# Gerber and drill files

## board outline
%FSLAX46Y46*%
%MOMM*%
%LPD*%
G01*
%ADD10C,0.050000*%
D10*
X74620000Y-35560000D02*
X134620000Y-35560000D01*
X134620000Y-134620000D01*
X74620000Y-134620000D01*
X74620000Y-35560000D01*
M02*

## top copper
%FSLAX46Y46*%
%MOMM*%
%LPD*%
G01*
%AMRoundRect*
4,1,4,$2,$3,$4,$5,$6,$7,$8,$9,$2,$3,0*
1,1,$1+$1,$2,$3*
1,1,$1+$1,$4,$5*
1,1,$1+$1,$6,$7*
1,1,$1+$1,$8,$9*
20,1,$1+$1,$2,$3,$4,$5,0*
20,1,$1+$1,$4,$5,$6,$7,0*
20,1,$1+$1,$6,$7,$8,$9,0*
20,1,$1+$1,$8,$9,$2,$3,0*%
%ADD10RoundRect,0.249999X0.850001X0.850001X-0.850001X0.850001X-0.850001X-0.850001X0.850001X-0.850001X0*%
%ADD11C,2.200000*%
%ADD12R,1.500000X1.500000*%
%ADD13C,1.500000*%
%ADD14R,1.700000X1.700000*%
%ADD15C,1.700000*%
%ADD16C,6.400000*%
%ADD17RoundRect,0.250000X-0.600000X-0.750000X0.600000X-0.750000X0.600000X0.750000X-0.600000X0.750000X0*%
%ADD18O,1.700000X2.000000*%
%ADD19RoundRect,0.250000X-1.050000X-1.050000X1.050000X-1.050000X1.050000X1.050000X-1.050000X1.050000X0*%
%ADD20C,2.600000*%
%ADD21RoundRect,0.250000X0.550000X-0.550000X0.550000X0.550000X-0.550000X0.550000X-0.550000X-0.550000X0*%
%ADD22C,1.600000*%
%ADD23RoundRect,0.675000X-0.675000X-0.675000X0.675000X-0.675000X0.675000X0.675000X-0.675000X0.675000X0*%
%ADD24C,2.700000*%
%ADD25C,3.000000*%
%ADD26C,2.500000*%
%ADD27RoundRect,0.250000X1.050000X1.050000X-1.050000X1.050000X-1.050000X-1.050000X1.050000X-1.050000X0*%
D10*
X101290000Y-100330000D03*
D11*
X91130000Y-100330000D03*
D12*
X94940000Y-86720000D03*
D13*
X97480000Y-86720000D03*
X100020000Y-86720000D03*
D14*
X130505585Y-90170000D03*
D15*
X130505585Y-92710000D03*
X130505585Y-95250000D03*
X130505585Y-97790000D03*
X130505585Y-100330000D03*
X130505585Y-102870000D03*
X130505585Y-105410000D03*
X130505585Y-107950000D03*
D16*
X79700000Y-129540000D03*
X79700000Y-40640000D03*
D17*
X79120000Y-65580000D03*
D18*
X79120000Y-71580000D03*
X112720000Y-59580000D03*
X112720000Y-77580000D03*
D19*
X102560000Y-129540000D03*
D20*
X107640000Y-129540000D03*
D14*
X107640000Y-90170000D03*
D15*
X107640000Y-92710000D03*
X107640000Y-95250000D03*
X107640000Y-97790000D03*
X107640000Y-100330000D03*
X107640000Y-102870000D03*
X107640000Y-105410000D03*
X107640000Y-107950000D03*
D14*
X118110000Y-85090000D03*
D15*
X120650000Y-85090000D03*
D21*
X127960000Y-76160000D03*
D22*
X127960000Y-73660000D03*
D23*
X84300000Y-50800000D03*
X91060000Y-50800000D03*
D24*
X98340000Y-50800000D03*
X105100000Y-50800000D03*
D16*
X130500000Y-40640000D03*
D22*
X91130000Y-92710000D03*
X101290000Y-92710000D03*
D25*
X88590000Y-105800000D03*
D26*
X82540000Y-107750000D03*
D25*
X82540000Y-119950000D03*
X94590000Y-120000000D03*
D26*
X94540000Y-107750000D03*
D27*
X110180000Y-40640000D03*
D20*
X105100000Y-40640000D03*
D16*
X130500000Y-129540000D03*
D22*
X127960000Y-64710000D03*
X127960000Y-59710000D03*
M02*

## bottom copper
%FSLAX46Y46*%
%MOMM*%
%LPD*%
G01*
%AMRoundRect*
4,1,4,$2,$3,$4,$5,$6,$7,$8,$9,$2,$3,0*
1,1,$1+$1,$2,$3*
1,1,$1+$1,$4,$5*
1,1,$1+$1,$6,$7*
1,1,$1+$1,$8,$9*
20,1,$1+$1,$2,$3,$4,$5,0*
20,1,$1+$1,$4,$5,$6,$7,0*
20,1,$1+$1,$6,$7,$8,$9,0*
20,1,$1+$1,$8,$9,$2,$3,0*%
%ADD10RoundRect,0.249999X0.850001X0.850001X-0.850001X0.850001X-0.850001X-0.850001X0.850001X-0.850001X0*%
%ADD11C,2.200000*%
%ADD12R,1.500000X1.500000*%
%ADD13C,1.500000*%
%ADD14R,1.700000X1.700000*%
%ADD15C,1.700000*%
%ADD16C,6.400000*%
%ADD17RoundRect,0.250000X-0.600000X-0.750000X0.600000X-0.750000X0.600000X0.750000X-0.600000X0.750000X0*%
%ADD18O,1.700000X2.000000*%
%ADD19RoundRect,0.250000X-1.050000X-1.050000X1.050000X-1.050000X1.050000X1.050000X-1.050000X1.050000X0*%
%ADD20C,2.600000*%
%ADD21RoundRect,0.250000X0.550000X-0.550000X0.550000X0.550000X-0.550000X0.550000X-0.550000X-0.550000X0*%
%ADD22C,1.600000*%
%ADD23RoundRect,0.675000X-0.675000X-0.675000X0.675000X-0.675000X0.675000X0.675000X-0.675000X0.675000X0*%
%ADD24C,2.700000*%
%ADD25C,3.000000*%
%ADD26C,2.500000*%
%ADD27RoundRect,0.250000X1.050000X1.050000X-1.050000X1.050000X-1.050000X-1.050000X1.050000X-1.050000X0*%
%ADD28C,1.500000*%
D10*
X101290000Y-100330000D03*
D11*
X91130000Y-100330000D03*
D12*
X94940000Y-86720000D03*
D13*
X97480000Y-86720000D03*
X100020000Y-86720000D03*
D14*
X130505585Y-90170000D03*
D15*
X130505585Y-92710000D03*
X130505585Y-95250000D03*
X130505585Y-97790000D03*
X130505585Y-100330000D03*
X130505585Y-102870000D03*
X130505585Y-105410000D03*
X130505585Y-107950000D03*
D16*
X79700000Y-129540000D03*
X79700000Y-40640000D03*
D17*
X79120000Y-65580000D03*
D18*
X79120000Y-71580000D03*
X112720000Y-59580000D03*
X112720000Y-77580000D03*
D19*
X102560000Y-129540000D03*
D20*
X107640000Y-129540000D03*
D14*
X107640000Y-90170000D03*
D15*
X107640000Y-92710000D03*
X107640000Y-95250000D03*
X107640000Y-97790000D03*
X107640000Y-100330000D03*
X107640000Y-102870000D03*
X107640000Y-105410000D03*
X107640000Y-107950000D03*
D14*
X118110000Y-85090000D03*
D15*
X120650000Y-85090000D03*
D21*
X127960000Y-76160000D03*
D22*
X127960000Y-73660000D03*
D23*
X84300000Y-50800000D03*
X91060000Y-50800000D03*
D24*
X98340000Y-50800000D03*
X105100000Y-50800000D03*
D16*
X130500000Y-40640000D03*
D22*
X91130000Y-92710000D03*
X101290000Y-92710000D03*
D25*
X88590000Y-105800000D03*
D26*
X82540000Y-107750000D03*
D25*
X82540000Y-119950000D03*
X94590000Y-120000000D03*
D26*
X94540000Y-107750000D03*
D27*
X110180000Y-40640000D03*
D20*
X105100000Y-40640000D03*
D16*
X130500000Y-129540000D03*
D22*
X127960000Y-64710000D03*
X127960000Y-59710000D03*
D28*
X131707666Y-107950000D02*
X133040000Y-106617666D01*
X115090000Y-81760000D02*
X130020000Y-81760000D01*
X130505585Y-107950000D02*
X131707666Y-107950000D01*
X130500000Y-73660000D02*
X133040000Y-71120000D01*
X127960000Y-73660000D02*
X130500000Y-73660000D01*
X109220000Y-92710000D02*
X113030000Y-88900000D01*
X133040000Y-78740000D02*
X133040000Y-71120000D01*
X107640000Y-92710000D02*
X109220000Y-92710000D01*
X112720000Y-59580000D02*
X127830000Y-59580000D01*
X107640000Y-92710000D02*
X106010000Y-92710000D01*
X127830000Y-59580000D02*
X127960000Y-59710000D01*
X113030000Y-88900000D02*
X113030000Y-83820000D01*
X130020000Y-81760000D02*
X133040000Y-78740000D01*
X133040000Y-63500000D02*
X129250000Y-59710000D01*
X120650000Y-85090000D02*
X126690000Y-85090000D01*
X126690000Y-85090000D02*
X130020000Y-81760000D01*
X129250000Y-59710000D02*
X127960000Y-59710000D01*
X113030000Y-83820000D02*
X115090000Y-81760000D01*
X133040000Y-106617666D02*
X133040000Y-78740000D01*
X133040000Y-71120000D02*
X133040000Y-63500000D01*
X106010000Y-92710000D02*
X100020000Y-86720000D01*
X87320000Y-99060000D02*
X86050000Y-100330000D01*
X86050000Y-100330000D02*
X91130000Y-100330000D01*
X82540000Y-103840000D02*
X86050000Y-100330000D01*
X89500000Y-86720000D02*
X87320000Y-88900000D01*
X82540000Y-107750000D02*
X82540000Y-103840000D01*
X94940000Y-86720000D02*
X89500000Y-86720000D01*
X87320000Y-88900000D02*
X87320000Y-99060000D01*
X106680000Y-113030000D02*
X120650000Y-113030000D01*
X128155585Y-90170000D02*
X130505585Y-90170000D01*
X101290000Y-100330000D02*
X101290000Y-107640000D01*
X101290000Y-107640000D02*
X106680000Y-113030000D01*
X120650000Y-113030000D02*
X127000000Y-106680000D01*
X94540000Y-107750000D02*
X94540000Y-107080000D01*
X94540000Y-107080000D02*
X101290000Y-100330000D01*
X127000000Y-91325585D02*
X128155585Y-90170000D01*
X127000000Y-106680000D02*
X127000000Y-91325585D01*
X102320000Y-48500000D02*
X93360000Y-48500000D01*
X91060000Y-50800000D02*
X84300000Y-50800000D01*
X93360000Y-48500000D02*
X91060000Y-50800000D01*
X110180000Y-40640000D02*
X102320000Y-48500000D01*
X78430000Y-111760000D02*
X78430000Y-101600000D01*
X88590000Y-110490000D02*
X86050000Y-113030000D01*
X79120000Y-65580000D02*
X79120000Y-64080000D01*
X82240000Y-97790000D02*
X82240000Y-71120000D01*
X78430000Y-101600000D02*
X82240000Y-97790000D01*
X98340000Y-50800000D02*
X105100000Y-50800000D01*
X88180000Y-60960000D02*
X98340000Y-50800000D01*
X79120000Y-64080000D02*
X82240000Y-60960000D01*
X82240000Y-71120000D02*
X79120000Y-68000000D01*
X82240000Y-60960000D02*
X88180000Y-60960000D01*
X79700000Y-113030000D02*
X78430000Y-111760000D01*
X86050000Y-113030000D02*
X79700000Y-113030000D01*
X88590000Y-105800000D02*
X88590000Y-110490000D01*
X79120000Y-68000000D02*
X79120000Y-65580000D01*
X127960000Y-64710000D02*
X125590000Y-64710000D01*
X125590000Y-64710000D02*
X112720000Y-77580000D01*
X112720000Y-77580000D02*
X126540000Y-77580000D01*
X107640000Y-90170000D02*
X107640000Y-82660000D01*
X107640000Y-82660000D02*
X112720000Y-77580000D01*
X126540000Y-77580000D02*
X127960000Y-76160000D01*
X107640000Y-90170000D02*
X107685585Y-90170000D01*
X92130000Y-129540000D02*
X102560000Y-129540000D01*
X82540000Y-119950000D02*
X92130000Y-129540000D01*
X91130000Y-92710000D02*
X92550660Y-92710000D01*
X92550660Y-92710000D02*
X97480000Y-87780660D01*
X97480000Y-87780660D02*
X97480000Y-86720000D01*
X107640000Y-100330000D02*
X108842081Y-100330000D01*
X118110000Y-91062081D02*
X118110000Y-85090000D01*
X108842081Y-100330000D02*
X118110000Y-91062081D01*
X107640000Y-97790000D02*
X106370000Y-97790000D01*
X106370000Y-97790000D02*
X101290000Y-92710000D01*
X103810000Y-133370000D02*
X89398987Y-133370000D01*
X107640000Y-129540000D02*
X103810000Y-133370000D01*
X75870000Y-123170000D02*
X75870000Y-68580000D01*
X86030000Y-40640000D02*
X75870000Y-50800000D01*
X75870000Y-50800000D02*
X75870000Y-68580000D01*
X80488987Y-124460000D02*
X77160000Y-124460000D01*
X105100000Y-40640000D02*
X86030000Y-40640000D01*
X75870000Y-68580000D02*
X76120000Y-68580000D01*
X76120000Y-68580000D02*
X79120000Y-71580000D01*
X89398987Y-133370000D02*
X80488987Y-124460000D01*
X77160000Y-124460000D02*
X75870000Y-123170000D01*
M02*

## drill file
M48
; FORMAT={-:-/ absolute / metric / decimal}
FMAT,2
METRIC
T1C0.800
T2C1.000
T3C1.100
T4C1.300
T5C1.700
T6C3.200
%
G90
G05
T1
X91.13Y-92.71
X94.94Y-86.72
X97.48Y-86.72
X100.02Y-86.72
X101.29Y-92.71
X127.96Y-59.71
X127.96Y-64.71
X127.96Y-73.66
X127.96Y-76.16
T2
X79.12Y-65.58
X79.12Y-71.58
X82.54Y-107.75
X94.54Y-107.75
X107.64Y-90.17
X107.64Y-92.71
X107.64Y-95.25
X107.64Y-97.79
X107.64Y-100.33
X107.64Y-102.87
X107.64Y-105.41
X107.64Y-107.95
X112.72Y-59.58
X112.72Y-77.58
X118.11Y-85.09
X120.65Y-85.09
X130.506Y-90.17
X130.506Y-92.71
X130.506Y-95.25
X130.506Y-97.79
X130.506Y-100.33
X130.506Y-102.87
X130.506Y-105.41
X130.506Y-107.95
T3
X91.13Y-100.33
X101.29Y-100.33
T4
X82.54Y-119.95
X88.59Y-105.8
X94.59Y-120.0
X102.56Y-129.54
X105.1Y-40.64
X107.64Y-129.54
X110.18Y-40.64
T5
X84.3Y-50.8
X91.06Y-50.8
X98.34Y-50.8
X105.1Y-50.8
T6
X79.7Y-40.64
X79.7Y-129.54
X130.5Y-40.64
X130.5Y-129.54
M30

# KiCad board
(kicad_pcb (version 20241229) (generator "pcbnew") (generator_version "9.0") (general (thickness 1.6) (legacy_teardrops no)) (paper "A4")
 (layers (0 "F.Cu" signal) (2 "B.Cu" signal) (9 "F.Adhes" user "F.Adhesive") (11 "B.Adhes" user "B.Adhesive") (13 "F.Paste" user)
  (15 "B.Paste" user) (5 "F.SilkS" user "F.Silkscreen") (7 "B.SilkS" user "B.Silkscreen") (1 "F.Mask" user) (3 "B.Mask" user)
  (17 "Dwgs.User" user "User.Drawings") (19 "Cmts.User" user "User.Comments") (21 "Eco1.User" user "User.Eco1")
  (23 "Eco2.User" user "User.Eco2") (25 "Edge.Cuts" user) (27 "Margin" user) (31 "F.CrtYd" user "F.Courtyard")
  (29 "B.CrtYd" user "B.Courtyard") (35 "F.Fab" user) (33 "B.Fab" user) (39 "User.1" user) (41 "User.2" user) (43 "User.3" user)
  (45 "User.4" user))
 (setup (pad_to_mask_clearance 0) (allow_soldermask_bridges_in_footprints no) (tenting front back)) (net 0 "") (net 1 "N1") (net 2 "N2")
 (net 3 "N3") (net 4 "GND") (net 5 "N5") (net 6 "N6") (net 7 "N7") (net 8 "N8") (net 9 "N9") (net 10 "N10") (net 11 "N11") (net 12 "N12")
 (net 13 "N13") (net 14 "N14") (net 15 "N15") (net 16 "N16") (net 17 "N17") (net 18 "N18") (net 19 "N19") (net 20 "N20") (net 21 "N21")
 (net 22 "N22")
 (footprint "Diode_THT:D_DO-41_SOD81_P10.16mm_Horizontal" (layer "F.Cu") (at 101.29 100.33 180)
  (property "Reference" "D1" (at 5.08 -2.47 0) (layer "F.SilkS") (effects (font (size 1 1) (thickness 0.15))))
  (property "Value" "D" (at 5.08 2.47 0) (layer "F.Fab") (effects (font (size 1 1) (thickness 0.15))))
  (pad "1" thru_hole roundrect (at 0 0 180) (size 2.2 2.2) (drill 1.1) (layers "*.Cu" "*.Mask") (remove_unused_layers no)
   (roundrect_rratio 0.113636) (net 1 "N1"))
  (pad "2" thru_hole circle (at 10.16 0 180) (size 2.2 2.2) (drill 1.1) (layers "*.Cu" "*.Mask") (remove_unused_layers no) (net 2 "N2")))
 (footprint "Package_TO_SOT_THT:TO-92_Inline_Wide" (layer "F.Cu") (at 94.94 86.72)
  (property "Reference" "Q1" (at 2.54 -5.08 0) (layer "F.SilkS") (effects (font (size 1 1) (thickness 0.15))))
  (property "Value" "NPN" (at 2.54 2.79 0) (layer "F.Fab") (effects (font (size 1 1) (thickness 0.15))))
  (pad "1" thru_hole rect (at 0 0) (size 1.5 1.5) (drill 0.8) (layers "*.Cu" "*.Mask") (remove_unused_layers no) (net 2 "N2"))
  (pad "2" thru_hole circle (at 2.54 0) (size 1.5 1.5) (drill 0.8) (layers "*.Cu" "*.Mask") (remove_unused_layers no) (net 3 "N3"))
  (pad "3" thru_hole circle (at 5.08 0) (size 1.5 1.5) (drill 0.8) (layers "*.Cu" "*.Mask") (remove_unused_layers no) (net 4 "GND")))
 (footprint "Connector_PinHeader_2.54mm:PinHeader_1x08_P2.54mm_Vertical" (layer "F.Cu") (at 130.505585 90.17)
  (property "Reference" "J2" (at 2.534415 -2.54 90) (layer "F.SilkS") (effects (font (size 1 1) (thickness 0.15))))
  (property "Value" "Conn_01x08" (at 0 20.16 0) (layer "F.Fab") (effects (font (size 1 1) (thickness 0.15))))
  (pad "1" thru_hole rect (at 0 0) (size 1.7 1.7) (drill 1) (layers "*.Cu" "*.Mask") (remove_unused_layers no) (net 1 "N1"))
  (pad "2" thru_hole circle (at 0 2.54) (size 1.7 1.7) (drill 1) (layers "*.Cu" "*.Mask") (remove_unused_layers no) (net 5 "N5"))
  (pad "3" thru_hole circle (at 0 5.08) (size 1.7 1.7) (drill 1) (layers "*.Cu" "*.Mask") (remove_unused_layers no) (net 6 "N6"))
  (pad "4" thru_hole circle (at 0 7.62) (size 1.7 1.7) (drill 1) (layers "*.Cu" "*.Mask") (remove_unused_layers no) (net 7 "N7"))
  (pad "5" thru_hole circle (at 0 10.16) (size 1.7 1.7) (drill 1) (layers "*.Cu" "*.Mask") (remove_unused_layers no) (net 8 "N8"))
  (pad "6" thru_hole circle (at 0 12.7) (size 1.7 1.7) (drill 1) (layers "*.Cu" "*.Mask") (remove_unused_layers no) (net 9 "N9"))
  (pad "7" thru_hole circle (at 0 15.24) (size 1.7 1.7) (drill 1) (layers "*.Cu" "*.Mask") (remove_unused_layers no) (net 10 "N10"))
  (pad "8" thru_hole circle (at 0 17.78) (size 1.7 1.7) (drill 1) (layers "*.Cu" "*.Mask") (remove_unused_layers no) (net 4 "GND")))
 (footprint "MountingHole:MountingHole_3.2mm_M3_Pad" (layer "F.Cu") (at 79.7 129.54)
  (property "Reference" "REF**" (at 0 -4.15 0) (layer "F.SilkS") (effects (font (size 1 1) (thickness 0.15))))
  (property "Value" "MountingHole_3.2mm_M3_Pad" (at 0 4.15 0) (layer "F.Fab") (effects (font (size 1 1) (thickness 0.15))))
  (pad "1" thru_hole circle (at 0 0) (size 6.4 6.4) (drill 3.2) (layers "*.Cu" "*.Mask") (remove_unused_layers no) (zone_connect 2)))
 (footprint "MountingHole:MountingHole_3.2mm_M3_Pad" (layer "F.Cu") (at 79.7 40.64)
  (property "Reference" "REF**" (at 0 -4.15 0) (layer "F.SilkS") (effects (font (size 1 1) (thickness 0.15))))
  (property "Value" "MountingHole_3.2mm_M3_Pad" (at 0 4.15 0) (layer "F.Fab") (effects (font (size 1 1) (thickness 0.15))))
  (pad "1" thru_hole circle (at 0 0) (size 6.4 6.4) (drill 3.2) (layers "*.Cu" "*.Mask") (remove_unused_layers no) (zone_connect 2)))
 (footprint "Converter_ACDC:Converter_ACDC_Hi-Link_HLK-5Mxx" (layer "F.Cu") (at 79.12 65.58)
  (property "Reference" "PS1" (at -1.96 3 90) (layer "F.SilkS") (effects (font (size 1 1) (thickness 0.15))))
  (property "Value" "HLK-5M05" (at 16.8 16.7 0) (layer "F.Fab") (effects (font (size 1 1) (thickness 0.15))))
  (pad "1" thru_hole roundrect (at 0 0) (size 1.7 2) (drill 1) (layers "*.Cu" "*.Mask") (remove_unused_layers no)
   (roundrect_rratio 0.147059) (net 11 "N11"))
  (pad "2" thru_hole oval (at 0 6) (size 1.7 2) (drill 1) (layers "*.Cu" "*.Mask") (remove_unused_layers no) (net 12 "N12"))
  (pad "3" thru_hole oval (at 33.6 -6) (size 1.7 2) (drill 1) (layers "*.Cu" "*.Mask") (remove_unused_layers no) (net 4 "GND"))
  (pad "4" thru_hole oval (at 33.6 12) (size 1.7 2) (drill 1) (layers "*.Cu" "*.Mask") (remove_unused_layers no) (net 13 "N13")))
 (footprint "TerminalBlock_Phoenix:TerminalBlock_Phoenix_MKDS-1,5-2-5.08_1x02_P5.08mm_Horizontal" (layer "F.Cu") (at 102.56 129.54)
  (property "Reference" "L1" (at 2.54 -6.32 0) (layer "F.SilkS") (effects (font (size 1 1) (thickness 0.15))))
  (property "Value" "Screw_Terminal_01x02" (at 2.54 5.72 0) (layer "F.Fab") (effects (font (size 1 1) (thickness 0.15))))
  (pad "1" thru_hole roundrect (at 0 0) (size 2.6 2.6) (drill 1.3) (layers "*.Cu" "*.Mask") (remove_unused_layers no)
   (roundrect_rratio 0.096154) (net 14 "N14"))
  (pad "2" thru_hole circle (at 5.08 0) (size 2.6 2.6) (drill 1.3) (layers "*.Cu" "*.Mask") (remove_unused_layers no) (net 12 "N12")))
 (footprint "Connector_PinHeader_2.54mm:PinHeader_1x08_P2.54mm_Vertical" (layer "F.Cu") (at 107.64 90.17)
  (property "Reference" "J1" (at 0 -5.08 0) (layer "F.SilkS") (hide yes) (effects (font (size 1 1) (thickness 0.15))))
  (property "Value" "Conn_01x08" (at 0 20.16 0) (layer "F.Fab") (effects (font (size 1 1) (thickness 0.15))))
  (pad "1" thru_hole rect (at 0 0) (size 1.7 1.7) (drill 1) (layers "*.Cu" "*.Mask") (remove_unused_layers no) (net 13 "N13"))
  (pad "2" thru_hole circle (at 0 2.54) (size 1.7 1.7) (drill 1) (layers "*.Cu" "*.Mask") (remove_unused_layers no) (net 4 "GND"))
  (pad "3" thru_hole circle (at 0 5.08) (size 1.7 1.7) (drill 1) (layers "*.Cu" "*.Mask") (remove_unused_layers no) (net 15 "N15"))
  (pad "4" thru_hole circle (at 0 7.62) (size 1.7 1.7) (drill 1) (layers "*.Cu" "*.Mask") (remove_unused_layers no) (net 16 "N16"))
  (pad "5" thru_hole circle (at 0 10.16) (size 1.7 1.7) (drill 1) (layers "*.Cu" "*.Mask") (remove_unused_layers no) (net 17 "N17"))
  (pad "6" thru_hole circle (at 0 12.7) (size 1.7 1.7) (drill 1) (layers "*.Cu" "*.Mask") (remove_unused_layers no) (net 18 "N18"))
  (pad "7" thru_hole circle (at 0 15.24) (size 1.7 1.7) (drill 1) (layers "*.Cu" "*.Mask") (remove_unused_layers no) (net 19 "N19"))
  (pad "8" thru_hole circle (at 0 17.78) (size 1.7 1.7) (drill 1) (layers "*.Cu" "*.Mask") (remove_unused_layers no) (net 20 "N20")))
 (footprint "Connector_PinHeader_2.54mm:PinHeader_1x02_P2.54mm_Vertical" (layer "F.Cu") (at 118.11 85.09 90)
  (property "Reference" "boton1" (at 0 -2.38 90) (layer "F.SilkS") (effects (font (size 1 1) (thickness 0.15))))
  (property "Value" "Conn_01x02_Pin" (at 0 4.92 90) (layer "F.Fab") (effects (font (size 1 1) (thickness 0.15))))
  (pad "1" thru_hole rect (at 0 0 90) (size 1.7 1.7) (drill 1) (layers "*.Cu" "*.Mask") (remove_unused_layers no) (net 17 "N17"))
  (pad "2" thru_hole circle (at 0 2.54 90) (size 1.7 1.7) (drill 1) (layers "*.Cu" "*.Mask") (remove_unused_layers no) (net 4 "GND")))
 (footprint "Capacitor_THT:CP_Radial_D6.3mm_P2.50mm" (layer "F.Cu") (at 127.96 76.16 90)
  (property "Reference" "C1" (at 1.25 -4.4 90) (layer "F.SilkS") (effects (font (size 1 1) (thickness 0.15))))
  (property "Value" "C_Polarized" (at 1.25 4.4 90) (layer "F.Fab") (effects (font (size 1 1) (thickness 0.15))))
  (pad "1" thru_hole roundrect (at 0 0 90) (size 1.6 1.6) (drill 0.8) (layers "*.Cu" "*.Mask") (remove_unused_layers no)
   (roundrect_rratio 0.15625) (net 13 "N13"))
  (pad "2" thru_hole circle (at 2.5 0 90) (size 1.6 1.6) (drill 0.8) (layers "*.Cu" "*.Mask") (remove_unused_layers no) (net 4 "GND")))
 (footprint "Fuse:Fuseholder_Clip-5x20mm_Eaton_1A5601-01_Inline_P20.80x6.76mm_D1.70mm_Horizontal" (layer "F.Cu") (at 84.3 50.8)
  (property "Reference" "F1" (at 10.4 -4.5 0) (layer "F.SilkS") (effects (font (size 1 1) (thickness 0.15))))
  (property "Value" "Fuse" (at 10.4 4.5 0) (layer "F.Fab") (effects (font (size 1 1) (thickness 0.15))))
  (pad "1" thru_hole roundrect (at 0 0) (size 2.7 2.7) (drill 1.7) (layers "*.Cu" "*.Mask") (remove_unused_layers no)
   (roundrect_rratio 0.25) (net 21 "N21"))
  (pad "1" thru_hole roundrect (at 6.76 0) (size 2.7 2.7) (drill 1.7) (layers "*.Cu" "*.Mask") (remove_unused_layers no)
   (roundrect_rratio 0.25) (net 21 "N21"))
  (pad "2" thru_hole circle (at 14.04 0) (size 2.7 2.7) (drill 1.7) (layers "*.Cu" "*.Mask") (remove_unused_layers no) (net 11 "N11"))
  (pad "2" thru_hole circle (at 20.8 0) (size 2.7 2.7) (drill 1.7) (layers "*.Cu" "*.Mask") (remove_unused_layers no) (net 11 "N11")))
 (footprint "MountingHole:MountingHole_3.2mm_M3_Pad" (layer "F.Cu") (at 130.5 40.64)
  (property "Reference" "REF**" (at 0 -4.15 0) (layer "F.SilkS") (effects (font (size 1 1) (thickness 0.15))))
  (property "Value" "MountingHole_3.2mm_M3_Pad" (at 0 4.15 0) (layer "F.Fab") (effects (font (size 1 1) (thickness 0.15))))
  (pad "1" thru_hole circle (at 0 0) (size 6.4 6.4) (drill 3.2) (layers "*.Cu" "*.Mask") (remove_unused_layers no) (zone_connect 2)))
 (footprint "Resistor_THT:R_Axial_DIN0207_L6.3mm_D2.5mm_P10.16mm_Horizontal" (layer "F.Cu") (at 91.13 92.71)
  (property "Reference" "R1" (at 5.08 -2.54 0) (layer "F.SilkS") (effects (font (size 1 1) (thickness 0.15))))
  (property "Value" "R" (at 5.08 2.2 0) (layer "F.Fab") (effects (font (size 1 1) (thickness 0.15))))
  (pad "1" thru_hole circle (at 0 0) (size 1.6 1.6) (drill 0.8) (layers "*.Cu" "*.Mask") (remove_unused_layers no) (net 3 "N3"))
  (pad "2" thru_hole circle (at 10.16 0) (size 1.6 1.6) (drill 0.8) (layers "*.Cu" "*.Mask") (remove_unused_layers no) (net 16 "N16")))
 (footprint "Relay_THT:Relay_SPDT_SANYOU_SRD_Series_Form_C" (layer "F.Cu") (at 88.59 105.8 -90)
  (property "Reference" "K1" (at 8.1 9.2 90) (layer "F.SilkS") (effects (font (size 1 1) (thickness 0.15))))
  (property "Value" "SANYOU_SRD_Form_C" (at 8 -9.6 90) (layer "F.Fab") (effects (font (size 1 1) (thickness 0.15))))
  (pad "1" thru_hole circle (at 0 0) (size 3 3) (drill 1.3) (layers "*.Cu" "*.Mask") (remove_unused_layers no) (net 11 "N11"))
  (pad "2" thru_hole circle (at 1.95 6.05) (size 2.5 2.5) (drill 1) (layers "*.Cu" "*.Mask") (remove_unused_layers no) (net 2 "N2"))
  (pad "3" thru_hole circle (at 14.15 6.05) (size 3 3) (drill 1.3) (layers "*.Cu" "*.Mask") (remove_unused_layers no) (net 14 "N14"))
  (pad "4" thru_hole circle (at 14.2 -6) (size 3 3) (drill 1.3) (layers "*.Cu" "*.Mask") (remove_unused_layers no) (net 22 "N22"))
  (pad "5" thru_hole circle (at 1.95 -5.95) (size 2.5 2.5) (drill 1) (layers "*.Cu" "*.Mask") (remove_unused_layers no) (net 1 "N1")))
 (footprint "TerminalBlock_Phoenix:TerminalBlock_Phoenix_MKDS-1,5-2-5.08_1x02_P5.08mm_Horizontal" (layer "F.Cu") (at 110.18 40.64 180)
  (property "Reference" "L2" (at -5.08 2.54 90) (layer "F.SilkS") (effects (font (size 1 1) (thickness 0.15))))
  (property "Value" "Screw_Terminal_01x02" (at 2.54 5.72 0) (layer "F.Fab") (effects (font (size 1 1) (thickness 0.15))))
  (pad "1" thru_hole roundrect (at 0 0 180) (size 2.6 2.6) (drill 1.3) (layers "*.Cu" "*.Mask") (remove_unused_layers no)
   (roundrect_rratio 0.096154) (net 21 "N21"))
  (pad "2" thru_hole circle (at 5.08 0 180) (size 2.6 2.6) (drill 1.3) (layers "*.Cu" "*.Mask") (remove_unused_layers no) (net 12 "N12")))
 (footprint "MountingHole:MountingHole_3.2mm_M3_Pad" (layer "F.Cu") (at 130.5 129.54)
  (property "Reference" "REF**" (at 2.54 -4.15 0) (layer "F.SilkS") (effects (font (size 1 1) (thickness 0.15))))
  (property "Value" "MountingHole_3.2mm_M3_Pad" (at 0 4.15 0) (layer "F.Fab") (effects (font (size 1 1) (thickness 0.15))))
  (pad "1" thru_hole circle (at 0 0) (size 6.4 6.4) (drill 3.2) (layers "*.Cu" "*.Mask") (remove_unused_layers no) (zone_connect 2)))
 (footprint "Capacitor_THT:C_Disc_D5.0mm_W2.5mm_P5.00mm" (layer "F.Cu") (at 127.96 64.71 90)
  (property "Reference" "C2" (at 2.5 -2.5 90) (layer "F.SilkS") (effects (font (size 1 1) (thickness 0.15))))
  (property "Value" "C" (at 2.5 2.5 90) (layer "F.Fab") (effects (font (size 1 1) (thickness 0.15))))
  (pad "1" thru_hole circle (at 0 0 90) (size 1.6 1.6) (drill 0.8) (layers "*.Cu" "*.Mask") (remove_unused_layers no) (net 13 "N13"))
  (pad "2" thru_hole circle (at 5 0 90) (size 1.6 1.6) (drill 0.8) (layers "*.Cu" "*.Mask") (remove_unused_layers no) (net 4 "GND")))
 (gr_rect (start 74.62 35.56) (end 134.62 134.62) (stroke (width 0.05) (type solid)) (fill no) (layer "Edge.Cuts"))
 (segment (start 131.707666 107.95) (end 133.04 106.617666) (width 1.5) (layer "B.Cu") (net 4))
 (segment (start 115.09 81.76) (end 130.02 81.76) (width 1.5) (layer "B.Cu") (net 4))
 (segment (start 130.505585 107.95) (end 131.707666 107.95) (width 1.5) (layer "B.Cu") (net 4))
 (segment (start 130.5 73.66) (end 133.04 71.12) (width 1.5) (layer "B.Cu") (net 4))
 (segment (start 127.96 73.66) (end 130.5 73.66) (width 1.5) (layer "B.Cu") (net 4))
 (segment (start 109.22 92.71) (end 113.03 88.9) (width 1.5) (layer "B.Cu") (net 4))
 (segment (start 133.04 78.74) (end 133.04 71.12) (width 1.5) (layer "B.Cu") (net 4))
 (segment (start 107.64 92.71) (end 109.22 92.71) (width 1.5) (layer "B.Cu") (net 4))
 (segment (start 112.72 59.58) (end 127.83 59.58) (width 1.5) (layer "B.Cu") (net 4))
 (segment (start 107.64 92.71) (end 106.01 92.71) (width 1.5) (layer "B.Cu") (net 4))
 (segment (start 127.83 59.58) (end 127.96 59.71) (width 1.5) (layer "B.Cu") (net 4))
 (segment (start 113.03 88.9) (end 113.03 83.82) (width 1.5) (layer "B.Cu") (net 4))
 (segment (start 130.02 81.76) (end 133.04 78.74) (width 1.5) (layer "B.Cu") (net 4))
 (segment (start 133.04 63.5) (end 129.25 59.71) (width 1.5) (layer "B.Cu") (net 4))
 (segment (start 120.65 85.09) (end 126.69 85.09) (width 1.5) (layer "B.Cu") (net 4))
 (segment (start 126.69 85.09) (end 130.02 81.76) (width 1.5) (layer "B.Cu") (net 4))
 (segment (start 129.25 59.71) (end 127.96 59.71) (width 1.5) (layer "B.Cu") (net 4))
 (segment (start 113.03 83.82) (end 115.09 81.76) (width 1.5) (layer "B.Cu") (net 4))
 (segment (start 133.04 106.617666) (end 133.04 78.74) (width 1.5) (layer "B.Cu") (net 4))
 (segment (start 133.04 71.12) (end 133.04 63.5) (width 1.5) (layer "B.Cu") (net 4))
 (segment (start 106.01 92.71) (end 100.02 86.72) (width 1.5) (layer "B.Cu") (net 4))
 (segment (start 87.32 99.06) (end 86.05 100.33) (width 1.5) (layer "B.Cu") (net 2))
 (segment (start 86.05 100.33) (end 91.13 100.33) (width 1.5) (layer "B.Cu") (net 2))
 (segment (start 82.54 103.84) (end 86.05 100.33) (width 1.5) (layer "B.Cu") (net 2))
 (segment (start 89.5 86.72) (end 87.32 88.9) (width 1.5) (layer "B.Cu") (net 2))
 (segment (start 82.54 107.75) (end 82.54 103.84) (width 1.5) (layer "B.Cu") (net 2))
 (segment (start 94.94 86.72) (end 89.5 86.72) (width 1.5) (layer "B.Cu") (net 2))
 (segment (start 87.32 88.9) (end 87.32 99.06) (width 1.5) (layer "B.Cu") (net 2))
 (segment (start 106.68 113.03) (end 120.65 113.03) (width 1.5) (layer "B.Cu") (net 1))
 (segment (start 128.155585 90.17) (end 130.505585 90.17) (width 1.5) (layer "B.Cu") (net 1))
 (segment (start 101.29 100.33) (end 101.29 107.64) (width 1.5) (layer "B.Cu") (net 1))
 (segment (start 101.29 107.64) (end 106.68 113.03) (width 1.5) (layer "B.Cu") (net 1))
 (segment (start 120.65 113.03) (end 127 106.68) (width 1.5) (layer "B.Cu") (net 1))
 (segment (start 94.54 107.75) (end 94.54 107.08) (width 1.5) (layer "B.Cu") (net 1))
 (segment (start 94.54 107.08) (end 101.29 100.33) (width 1.5) (layer "B.Cu") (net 1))
 (segment (start 127 91.325585) (end 128.155585 90.17) (width 1.5) (layer "B.Cu") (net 1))
 (segment (start 127 106.68) (end 127 91.325585) (width 1.5) (layer "B.Cu") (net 1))
 (segment (start 102.32 48.5) (end 93.36 48.5) (width 1.5) (layer "B.Cu") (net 21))
 (segment (start 91.06 50.8) (end 84.3 50.8) (width 1.5) (layer "B.Cu") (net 21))
 (segment (start 93.36 48.5) (end 91.06 50.8) (width 1.5) (layer "B.Cu") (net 21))
 (segment (start 110.18 40.64) (end 102.32 48.5) (width 1.5) (layer "B.Cu") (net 21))
 (segment (start 78.43 111.76) (end 78.43 101.6) (width 1.5) (layer "B.Cu") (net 11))
 (segment (start 88.59 110.49) (end 86.05 113.03) (width 1.5) (layer "B.Cu") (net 11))
 (segment (start 79.12 65.58) (end 79.12 64.08) (width 1.5) (layer "B.Cu") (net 11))
 (segment (start 82.24 97.79) (end 82.24 71.12) (width 1.5) (layer "B.Cu") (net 11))
 (segment (start 78.43 101.6) (end 82.24 97.79) (width 1.5) (layer "B.Cu") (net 11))
 (segment (start 98.34 50.8) (end 105.1 50.8) (width 1.5) (layer "B.Cu") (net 11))
 (segment (start 88.18 60.96) (end 98.34 50.8) (width 1.5) (layer "B.Cu") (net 11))
 (segment (start 79.12 64.08) (end 82.24 60.96) (width 1.5) (layer "B.Cu") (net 11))
 (segment (start 82.24 71.12) (end 79.12 68) (width 1.5) (layer "B.Cu") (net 11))
 (segment (start 82.24 60.96) (end 88.18 60.96) (width 1.5) (layer "B.Cu") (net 11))
 (segment (start 79.7 113.03) (end 78.43 111.76) (width 1.5) (layer "B.Cu") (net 11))
 (segment (start 86.05 113.03) (end 79.7 113.03) (width 1.5) (layer "B.Cu") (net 11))
 (segment (start 88.59 105.8) (end 88.59 110.49) (width 1.5) (layer "B.Cu") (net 11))
 (segment (start 79.12 68) (end 79.12 65.58) (width 1.5) (layer "B.Cu") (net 11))
 (segment (start 127.96 64.71) (end 125.59 64.71) (width 1.5) (layer "B.Cu") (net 13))
 (segment (start 125.59 64.71) (end 112.72 77.58) (width 1.5) (layer "B.Cu") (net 13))
 (segment (start 112.72 77.58) (end 126.54 77.58) (width 1.5) (layer "B.Cu") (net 13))
 (segment (start 107.64 90.17) (end 107.64 82.66) (width 1.5) (layer "B.Cu") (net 13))
 (segment (start 107.64 82.66) (end 112.72 77.58) (width 1.5) (layer "B.Cu") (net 13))
 (segment (start 126.54 77.58) (end 127.96 76.16) (width 1.5) (layer "B.Cu") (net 13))
 (segment (start 107.64 90.17) (end 107.685585 90.17) (width 1.5) (layer "B.Cu") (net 13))
 (segment (start 92.13 129.54) (end 102.56 129.54) (width 1.5) (layer "B.Cu") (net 14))
 (segment (start 82.54 119.95) (end 92.13 129.54) (width 1.5) (layer "B.Cu") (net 14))
 (segment (start 91.13 92.71) (end 92.55066 92.71) (width 1.5) (layer "B.Cu") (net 3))
 (segment (start 92.55066 92.71) (end 97.48 87.78066) (width 1.5) (layer "B.Cu") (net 3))
 (segment (start 97.48 87.78066) (end 97.48 86.72) (width 1.5) (layer "B.Cu") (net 3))
 (segment (start 107.64 100.33) (end 108.842081 100.33) (width 1.5) (layer "B.Cu") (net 17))
 (segment (start 118.11 91.062081) (end 118.11 85.09) (width 1.5) (layer "B.Cu") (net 17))
 (segment (start 108.842081 100.33) (end 118.11 91.062081) (width 1.5) (layer "B.Cu") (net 17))
 (segment (start 107.64 97.79) (end 106.37 97.79) (width 1.5) (layer "B.Cu") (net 16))
 (segment (start 106.37 97.79) (end 101.29 92.71) (width 1.5) (layer "B.Cu") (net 16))
 (segment (start 103.81 133.37) (end 89.398987 133.37) (width 1.5) (layer "B.Cu") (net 12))
 (segment (start 107.64 129.54) (end 103.81 133.37) (width 1.5) (layer "B.Cu") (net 12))
 (segment (start 75.87 123.17) (end 75.87 68.58) (width 1.5) (layer "B.Cu") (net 12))
 (segment (start 86.03 40.64) (end 75.87 50.8) (width 1.5) (layer "B.Cu") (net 12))
 (segment (start 75.87 50.8) (end 75.87 68.58) (width 1.5) (layer "B.Cu") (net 12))
 (segment (start 80.488987 124.46) (end 77.16 124.46) (width 1.5) (layer "B.Cu") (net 12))
 (segment (start 105.1 40.64) (end 86.03 40.64) (width 1.5) (layer "B.Cu") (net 12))
 (segment (start 75.87 68.58) (end 76.12 68.58) (width 1.5) (layer "B.Cu") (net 12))
 (segment (start 76.12 68.58) (end 79.12 71.58) (width 1.5) (layer "B.Cu") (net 12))
 (segment (start 89.398987 133.37) (end 80.488987 124.46) (width 1.5) (layer "B.Cu") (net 12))
 (segment (start 77.16 124.46) (end 75.87 123.17) (width 1.5) (layer "B.Cu") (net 12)))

